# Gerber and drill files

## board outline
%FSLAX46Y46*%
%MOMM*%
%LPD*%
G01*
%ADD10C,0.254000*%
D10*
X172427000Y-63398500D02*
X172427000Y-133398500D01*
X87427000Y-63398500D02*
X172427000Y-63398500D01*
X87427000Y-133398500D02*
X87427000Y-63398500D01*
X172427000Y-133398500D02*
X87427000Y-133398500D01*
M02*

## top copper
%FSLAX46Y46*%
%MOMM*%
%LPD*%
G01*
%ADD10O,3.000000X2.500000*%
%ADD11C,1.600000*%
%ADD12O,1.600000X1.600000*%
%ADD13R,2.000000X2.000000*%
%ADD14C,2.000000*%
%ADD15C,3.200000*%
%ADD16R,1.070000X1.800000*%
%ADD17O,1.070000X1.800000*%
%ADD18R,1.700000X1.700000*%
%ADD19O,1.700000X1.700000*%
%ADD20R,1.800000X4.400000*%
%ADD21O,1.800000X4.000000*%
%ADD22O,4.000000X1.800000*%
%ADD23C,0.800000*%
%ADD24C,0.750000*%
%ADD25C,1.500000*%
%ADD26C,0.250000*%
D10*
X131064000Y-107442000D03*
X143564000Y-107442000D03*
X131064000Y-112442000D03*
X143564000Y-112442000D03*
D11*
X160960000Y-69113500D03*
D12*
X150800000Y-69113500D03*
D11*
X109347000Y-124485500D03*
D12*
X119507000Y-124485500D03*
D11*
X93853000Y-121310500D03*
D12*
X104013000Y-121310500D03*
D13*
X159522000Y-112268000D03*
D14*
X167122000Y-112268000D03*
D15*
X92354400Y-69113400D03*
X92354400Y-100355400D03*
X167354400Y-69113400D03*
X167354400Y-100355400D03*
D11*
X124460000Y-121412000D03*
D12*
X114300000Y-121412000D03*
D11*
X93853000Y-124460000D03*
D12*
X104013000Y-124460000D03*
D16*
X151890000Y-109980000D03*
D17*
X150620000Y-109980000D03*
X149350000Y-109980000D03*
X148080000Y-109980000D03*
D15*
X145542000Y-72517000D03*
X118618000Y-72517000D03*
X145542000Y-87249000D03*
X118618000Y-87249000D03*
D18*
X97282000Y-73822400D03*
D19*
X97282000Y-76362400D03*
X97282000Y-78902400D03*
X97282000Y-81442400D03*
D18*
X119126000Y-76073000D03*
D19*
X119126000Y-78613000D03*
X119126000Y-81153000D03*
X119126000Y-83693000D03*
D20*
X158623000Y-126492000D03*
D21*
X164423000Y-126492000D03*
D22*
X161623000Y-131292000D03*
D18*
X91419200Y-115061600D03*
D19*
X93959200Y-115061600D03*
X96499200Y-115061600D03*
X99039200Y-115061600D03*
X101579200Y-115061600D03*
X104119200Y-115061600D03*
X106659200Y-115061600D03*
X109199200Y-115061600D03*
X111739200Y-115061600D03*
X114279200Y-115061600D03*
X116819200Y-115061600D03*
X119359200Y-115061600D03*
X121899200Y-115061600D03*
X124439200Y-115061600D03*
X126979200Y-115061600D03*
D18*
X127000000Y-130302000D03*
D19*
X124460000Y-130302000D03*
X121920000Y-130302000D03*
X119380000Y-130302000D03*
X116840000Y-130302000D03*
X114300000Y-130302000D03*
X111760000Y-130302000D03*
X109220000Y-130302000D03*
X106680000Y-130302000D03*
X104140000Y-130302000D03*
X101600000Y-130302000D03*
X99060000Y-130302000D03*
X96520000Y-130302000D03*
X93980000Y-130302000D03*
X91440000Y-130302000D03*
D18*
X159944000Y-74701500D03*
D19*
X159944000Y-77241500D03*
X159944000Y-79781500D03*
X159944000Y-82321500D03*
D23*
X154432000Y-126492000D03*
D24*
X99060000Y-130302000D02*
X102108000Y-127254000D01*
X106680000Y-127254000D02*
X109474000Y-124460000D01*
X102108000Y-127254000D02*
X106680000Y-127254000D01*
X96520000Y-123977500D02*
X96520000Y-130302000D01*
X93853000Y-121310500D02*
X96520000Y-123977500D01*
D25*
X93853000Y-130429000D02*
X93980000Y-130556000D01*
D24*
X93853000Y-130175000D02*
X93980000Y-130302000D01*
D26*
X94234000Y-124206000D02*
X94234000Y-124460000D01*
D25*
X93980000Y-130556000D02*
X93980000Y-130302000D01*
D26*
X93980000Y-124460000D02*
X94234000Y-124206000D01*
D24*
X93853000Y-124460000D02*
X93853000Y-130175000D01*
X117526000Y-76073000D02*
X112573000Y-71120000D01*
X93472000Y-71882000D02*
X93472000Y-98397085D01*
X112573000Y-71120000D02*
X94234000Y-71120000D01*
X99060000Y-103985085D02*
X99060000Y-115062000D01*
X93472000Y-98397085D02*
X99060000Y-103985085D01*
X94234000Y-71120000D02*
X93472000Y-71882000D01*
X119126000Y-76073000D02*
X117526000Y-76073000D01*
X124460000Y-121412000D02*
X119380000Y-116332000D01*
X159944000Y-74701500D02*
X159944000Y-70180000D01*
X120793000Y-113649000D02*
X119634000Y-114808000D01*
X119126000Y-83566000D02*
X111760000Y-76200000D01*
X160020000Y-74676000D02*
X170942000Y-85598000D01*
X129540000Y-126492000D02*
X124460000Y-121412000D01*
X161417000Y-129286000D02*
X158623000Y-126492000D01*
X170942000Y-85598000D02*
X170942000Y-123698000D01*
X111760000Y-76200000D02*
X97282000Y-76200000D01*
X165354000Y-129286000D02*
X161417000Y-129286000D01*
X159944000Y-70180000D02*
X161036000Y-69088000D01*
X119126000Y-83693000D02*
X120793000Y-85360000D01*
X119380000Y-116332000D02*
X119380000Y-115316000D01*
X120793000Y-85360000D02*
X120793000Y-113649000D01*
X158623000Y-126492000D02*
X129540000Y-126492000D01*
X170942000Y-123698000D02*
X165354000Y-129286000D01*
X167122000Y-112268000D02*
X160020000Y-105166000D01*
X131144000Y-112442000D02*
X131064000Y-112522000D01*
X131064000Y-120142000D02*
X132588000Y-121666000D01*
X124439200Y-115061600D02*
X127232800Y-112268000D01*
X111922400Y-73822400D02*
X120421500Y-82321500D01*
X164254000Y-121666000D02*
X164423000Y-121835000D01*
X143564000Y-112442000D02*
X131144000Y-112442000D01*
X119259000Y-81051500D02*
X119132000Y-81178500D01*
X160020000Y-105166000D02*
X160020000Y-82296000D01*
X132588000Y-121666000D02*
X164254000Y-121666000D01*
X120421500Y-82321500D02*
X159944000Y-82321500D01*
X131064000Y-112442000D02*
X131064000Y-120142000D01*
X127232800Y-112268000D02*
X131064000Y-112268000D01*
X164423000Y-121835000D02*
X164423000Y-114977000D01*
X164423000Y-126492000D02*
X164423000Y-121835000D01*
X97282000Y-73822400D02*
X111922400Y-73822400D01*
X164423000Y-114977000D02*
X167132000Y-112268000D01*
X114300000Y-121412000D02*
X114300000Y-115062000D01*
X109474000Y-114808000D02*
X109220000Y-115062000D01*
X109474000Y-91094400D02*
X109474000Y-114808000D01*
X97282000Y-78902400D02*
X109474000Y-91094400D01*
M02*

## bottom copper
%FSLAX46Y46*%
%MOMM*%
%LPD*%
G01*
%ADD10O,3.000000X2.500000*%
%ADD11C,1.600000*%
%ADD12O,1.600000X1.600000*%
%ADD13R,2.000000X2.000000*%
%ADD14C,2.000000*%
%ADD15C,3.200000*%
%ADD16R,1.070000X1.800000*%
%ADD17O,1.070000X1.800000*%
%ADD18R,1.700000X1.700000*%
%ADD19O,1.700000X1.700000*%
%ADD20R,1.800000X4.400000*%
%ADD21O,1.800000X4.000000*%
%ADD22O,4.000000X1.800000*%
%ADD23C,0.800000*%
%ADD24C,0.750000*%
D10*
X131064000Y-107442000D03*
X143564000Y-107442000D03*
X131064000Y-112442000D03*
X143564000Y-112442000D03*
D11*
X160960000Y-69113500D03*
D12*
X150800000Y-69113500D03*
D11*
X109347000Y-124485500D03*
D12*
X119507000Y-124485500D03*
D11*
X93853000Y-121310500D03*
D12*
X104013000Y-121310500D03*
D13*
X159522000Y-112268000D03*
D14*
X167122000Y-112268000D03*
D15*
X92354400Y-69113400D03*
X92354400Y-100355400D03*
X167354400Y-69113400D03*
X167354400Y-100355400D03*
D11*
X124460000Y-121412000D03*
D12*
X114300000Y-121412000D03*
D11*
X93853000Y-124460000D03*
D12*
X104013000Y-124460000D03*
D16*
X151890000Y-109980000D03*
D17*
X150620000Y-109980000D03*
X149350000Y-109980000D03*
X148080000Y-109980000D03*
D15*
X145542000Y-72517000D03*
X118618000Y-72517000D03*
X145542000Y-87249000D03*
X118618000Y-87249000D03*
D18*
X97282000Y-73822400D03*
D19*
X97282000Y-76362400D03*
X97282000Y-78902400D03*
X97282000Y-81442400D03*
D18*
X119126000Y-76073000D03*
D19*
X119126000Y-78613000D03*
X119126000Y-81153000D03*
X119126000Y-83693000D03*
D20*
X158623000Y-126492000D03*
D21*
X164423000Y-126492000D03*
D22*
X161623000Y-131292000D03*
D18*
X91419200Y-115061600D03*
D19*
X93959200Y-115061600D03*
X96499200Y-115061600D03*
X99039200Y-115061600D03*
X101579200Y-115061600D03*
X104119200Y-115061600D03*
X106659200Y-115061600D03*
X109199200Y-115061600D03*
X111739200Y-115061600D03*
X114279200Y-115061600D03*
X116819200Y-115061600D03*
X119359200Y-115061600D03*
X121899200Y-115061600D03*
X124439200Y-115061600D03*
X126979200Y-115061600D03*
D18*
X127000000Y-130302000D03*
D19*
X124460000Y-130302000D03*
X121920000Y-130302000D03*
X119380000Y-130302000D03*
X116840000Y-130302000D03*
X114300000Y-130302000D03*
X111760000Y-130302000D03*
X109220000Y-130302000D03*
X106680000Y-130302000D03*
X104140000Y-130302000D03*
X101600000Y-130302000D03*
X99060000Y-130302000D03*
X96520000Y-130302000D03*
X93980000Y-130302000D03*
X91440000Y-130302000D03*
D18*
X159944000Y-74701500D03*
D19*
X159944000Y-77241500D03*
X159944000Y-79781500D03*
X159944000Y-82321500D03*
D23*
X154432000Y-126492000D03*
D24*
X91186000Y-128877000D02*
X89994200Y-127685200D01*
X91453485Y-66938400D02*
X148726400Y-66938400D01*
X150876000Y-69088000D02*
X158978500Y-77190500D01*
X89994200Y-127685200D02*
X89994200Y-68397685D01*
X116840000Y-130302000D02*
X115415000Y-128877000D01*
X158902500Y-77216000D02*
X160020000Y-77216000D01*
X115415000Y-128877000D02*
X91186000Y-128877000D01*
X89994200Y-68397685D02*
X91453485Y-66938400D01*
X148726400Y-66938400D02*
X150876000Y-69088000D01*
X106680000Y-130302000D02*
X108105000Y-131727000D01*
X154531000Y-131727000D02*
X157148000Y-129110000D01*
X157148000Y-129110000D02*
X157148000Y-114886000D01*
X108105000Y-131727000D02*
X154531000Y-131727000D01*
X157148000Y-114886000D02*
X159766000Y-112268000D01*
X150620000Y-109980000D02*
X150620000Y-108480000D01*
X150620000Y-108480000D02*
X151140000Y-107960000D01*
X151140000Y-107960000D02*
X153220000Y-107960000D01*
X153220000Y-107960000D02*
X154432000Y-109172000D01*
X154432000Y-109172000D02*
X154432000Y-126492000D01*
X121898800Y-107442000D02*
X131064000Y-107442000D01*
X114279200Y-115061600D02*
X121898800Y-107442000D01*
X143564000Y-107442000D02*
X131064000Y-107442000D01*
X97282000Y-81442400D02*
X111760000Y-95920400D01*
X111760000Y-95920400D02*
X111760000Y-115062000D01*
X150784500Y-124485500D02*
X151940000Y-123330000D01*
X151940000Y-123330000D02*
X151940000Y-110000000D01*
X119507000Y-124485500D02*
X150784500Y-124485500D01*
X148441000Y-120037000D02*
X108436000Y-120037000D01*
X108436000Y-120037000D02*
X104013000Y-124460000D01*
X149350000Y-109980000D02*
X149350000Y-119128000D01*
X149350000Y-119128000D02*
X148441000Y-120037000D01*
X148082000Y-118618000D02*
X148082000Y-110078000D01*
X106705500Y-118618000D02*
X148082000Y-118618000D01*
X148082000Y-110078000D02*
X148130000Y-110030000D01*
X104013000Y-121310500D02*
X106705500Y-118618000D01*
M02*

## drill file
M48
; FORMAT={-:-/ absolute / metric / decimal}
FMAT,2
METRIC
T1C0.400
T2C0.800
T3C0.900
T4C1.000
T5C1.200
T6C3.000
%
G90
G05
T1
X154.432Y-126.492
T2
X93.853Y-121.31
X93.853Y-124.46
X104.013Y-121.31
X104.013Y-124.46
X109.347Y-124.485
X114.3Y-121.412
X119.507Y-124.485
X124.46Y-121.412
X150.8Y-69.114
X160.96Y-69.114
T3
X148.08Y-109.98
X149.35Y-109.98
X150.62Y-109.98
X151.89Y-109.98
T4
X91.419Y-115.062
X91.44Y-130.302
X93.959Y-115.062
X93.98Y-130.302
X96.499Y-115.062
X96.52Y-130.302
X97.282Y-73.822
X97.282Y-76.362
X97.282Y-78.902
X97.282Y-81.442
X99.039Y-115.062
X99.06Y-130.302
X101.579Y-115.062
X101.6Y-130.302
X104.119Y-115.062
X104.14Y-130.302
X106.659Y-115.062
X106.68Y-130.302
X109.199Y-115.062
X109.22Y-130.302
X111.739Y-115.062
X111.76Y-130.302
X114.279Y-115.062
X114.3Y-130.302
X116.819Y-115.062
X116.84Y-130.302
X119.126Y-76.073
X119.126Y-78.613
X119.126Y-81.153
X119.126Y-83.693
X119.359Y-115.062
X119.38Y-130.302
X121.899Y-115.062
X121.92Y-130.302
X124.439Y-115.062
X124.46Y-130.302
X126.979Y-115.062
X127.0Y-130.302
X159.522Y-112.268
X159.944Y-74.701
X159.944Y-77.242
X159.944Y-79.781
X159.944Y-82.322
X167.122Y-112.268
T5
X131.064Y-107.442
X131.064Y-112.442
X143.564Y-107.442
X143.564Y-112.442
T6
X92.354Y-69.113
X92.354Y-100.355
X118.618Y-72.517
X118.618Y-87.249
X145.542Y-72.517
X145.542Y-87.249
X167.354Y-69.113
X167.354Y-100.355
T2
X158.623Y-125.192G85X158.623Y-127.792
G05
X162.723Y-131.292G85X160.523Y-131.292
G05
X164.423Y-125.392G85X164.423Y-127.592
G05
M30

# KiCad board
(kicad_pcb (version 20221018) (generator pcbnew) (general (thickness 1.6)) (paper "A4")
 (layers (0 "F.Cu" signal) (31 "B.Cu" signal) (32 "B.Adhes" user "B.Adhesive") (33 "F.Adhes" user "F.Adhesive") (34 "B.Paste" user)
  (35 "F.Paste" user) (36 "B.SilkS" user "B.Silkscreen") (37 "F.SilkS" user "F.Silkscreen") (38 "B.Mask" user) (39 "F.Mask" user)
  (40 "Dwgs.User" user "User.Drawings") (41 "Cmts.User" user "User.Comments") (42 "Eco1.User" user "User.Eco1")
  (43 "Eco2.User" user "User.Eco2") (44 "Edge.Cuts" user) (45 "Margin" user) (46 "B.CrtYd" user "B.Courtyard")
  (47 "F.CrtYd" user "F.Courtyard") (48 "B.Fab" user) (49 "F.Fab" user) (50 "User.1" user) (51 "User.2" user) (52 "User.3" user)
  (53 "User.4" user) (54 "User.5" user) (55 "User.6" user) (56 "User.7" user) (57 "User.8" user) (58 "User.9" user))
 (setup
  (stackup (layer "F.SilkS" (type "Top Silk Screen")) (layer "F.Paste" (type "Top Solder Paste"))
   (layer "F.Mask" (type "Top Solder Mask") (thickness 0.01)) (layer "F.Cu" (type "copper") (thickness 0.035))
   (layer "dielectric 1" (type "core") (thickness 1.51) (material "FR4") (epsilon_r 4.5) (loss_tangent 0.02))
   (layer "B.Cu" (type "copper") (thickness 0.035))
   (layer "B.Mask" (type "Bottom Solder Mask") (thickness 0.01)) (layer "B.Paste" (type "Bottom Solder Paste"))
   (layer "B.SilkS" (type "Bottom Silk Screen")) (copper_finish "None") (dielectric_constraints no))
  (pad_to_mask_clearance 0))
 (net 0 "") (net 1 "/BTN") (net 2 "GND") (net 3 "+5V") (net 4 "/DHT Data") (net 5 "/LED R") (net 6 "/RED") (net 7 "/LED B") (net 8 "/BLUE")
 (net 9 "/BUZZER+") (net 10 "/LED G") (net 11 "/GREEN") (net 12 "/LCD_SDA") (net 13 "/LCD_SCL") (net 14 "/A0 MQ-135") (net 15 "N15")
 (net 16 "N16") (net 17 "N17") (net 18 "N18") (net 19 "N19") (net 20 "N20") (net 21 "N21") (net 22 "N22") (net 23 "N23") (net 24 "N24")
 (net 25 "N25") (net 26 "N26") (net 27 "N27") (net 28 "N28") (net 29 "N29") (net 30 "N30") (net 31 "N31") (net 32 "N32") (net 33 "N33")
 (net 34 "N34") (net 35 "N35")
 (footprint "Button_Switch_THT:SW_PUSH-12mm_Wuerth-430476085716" (layer "F.Cu") (at 131.064 107.442)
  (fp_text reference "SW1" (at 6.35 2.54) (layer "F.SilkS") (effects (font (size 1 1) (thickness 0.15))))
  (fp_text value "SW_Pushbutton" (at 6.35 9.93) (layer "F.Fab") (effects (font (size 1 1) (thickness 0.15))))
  (pad "1" thru_hole oval (at 0 0) (size 3 2.5) (drill 1.2) (layers "*.Cu" "*.Mask") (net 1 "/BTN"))
  (pad "1" thru_hole oval (at 12.5 0) (size 3 2.5) (drill 1.2) (layers "*.Cu" "*.Mask") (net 1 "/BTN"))
  (pad "2" thru_hole oval (at 0 5) (size 3 2.5) (drill 1.2) (layers "*.Cu" "*.Mask") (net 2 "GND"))
  (pad "2" thru_hole oval (at 12.5 5) (size 3 2.5) (drill 1.2) (layers "*.Cu" "*.Mask") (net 2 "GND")))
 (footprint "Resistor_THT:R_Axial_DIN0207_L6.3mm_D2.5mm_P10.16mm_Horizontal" (layer "F.Cu") (at 160.96 69.1135 180)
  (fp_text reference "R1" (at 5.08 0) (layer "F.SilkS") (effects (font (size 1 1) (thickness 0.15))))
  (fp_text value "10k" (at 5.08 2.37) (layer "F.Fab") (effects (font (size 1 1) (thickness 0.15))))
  (pad "1" thru_hole circle (at 0 0 180) (size 1.6 1.6) (drill 0.8) (layers "*.Cu" "*.Mask") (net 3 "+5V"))
  (pad "2" thru_hole oval (at 10.16 0 180) (size 1.6 1.6) (drill 0.8) (layers "*.Cu" "*.Mask") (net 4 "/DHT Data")))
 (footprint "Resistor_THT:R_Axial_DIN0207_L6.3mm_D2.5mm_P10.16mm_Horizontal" (layer "F.Cu") (at 109.347 124.4855)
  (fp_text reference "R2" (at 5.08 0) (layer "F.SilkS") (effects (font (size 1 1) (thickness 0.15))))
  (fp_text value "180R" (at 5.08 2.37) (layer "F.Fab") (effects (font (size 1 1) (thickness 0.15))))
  (pad "1" thru_hole circle (at 0 0) (size 1.6 1.6) (drill 0.8) (layers "*.Cu" "*.Mask") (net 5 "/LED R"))
  (pad "2" thru_hole oval (at 10.16 0) (size 1.6 1.6) (drill 0.8) (layers "*.Cu" "*.Mask") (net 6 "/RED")))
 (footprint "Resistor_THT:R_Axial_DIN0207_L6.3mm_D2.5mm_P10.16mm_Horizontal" (layer "F.Cu") (at 93.853 121.3105)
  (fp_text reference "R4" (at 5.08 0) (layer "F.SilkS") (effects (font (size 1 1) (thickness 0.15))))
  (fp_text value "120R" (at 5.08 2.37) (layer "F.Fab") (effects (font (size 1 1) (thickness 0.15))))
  (pad "1" thru_hole circle (at 0 0) (size 1.6 1.6) (drill 0.8) (layers "*.Cu" "*.Mask") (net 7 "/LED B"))
  (pad "2" thru_hole oval (at 10.16 0) (size 1.6 1.6) (drill 0.8) (layers "*.Cu" "*.Mask") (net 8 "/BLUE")))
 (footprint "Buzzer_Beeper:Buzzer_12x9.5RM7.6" (layer "F.Cu") (at 159.522 112.268)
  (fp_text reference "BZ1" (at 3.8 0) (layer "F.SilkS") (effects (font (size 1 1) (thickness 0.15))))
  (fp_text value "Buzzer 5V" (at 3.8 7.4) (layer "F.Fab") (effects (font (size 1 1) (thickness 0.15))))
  (pad "1" thru_hole rect (at 0 0) (size 2 2) (drill 1) (layers "*.Cu" "*.Mask") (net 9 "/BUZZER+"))
  (pad "2" thru_hole circle (at 7.6 0) (size 2 2) (drill 1) (layers "*.Cu" "*.Mask") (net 2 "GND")))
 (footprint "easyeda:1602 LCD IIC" (layer "F.Cu") (at 89.8144 66.8274)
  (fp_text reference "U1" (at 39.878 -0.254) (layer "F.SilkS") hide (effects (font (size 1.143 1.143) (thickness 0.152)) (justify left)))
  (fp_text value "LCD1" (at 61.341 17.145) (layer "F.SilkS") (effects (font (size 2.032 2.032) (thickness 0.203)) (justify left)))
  (pad "" thru_hole circle (at 2.54 2.286) (size 3.2 3.2) (drill 3) (layers "*.Cu" "*.Mask"))
  (pad "" thru_hole circle (at 2.54 33.528) (size 3.2 3.2) (drill 3) (layers "*.Cu" "*.Mask"))
  (pad "" thru_hole circle (at 77.54 2.286) (size 3.2 3.2) (drill 3) (layers "*.Cu" "*.Mask"))
  (pad "" thru_hole circle (at 77.54 33.528) (size 3.2 3.2) (drill 3) (layers "*.Cu" "*.Mask")))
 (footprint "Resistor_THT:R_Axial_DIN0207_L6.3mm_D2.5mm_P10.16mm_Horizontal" (layer "F.Cu") (at 124.46 121.412 180)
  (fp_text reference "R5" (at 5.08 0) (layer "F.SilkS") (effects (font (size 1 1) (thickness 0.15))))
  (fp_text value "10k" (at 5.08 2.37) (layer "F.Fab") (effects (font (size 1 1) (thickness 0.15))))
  (pad "1" thru_hole circle (at 0 0 180) (size 1.6 1.6) (drill 0.8) (layers "*.Cu" "*.Mask") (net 3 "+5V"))
  (pad "2" thru_hole oval (at 10.16 0 180) (size 1.6 1.6) (drill 0.8) (layers "*.Cu" "*.Mask") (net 1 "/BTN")))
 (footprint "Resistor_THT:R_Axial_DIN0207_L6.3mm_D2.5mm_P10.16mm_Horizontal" (layer "F.Cu") (at 93.853 124.46)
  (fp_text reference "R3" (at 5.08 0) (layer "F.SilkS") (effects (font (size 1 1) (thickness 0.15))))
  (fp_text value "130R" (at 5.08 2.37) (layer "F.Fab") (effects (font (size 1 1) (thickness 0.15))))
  (pad "1" thru_hole circle (at 0 0) (size 1.6 1.6) (drill 0.8) (layers "*.Cu" "*.Mask") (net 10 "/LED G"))
  (pad "2" thru_hole oval (at 10.16 0) (size 1.6 1.6) (drill 0.8) (layers "*.Cu" "*.Mask") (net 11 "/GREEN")))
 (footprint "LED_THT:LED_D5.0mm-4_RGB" (layer "F.Cu") (at 151.89 109.98 180)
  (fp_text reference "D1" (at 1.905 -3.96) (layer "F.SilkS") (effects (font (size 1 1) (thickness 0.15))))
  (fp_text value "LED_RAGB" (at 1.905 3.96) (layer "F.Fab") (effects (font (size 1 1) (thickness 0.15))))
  (pad "1" thru_hole rect (at 0 0 180) (size 1.07 1.8) (drill 0.9) (layers "*.Cu" "*.Mask") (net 6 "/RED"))
  (pad "2" thru_hole oval (at 1.27 0 180) (size 1.07 1.8) (drill 0.9) (layers "*.Cu" "*.Mask") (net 3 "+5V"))
  (pad "3" thru_hole oval (at 2.54 0 180) (size 1.07 1.8) (drill 0.9) (layers "*.Cu" "*.Mask") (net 11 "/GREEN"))
  (pad "4" thru_hole oval (at 3.81 0 180) (size 1.07 1.8) (drill 0.9) (layers "*.Cu" "*.Mask") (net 8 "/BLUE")))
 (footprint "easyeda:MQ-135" (layer "F.Cu") (at 118.618 87.249 -90)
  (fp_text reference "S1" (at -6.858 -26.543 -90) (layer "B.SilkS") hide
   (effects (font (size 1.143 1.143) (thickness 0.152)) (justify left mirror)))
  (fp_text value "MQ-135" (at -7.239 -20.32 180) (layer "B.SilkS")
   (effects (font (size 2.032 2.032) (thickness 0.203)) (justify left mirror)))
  (pad "" thru_hole circle (at -14.732 -26.924) (size 3.2 3.2) (drill 3) (layers "*.Cu" "*.Mask"))
  (pad "" thru_hole circle (at -14.732 0) (size 3.2 3.2) (drill 3) (layers "*.Cu" "*.Mask"))
  (pad "" thru_hole circle (at 0 -26.924) (size 3.2 3.2) (drill 3) (layers "*.Cu" "*.Mask"))
  (pad "" thru_hole circle (at 0 0) (size 3.2 3.2) (drill 3) (layers "*.Cu" "*.Mask")))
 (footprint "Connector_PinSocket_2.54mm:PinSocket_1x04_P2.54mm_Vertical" (layer "F.Cu") (at 97.282 73.8224)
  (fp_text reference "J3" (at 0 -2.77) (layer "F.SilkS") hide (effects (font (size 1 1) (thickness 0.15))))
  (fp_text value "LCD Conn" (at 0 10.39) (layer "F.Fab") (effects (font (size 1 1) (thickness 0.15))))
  (pad "1" thru_hole rect (at 0 0) (size 1.7 1.7) (drill 1) (layers "*.Cu" "*.Mask") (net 2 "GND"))
  (pad "2" thru_hole oval (at 0 2.54) (size 1.7 1.7) (drill 1) (layers "*.Cu" "*.Mask") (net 3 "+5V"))
  (pad "3" thru_hole oval (at 0 5.08) (size 1.7 1.7) (drill 1) (layers "*.Cu" "*.Mask") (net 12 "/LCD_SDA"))
  (pad "4" thru_hole oval (at 0 7.62) (size 1.7 1.7) (drill 1) (layers "*.Cu" "*.Mask") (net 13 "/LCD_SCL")))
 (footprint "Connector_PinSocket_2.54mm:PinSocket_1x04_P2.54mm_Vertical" (layer "B.Cu") (at 119.126 76.073 180)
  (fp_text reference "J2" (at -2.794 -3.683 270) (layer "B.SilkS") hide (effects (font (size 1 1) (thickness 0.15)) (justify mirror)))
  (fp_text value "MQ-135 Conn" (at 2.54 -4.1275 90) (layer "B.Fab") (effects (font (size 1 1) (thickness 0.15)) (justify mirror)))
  (pad "1" thru_hole rect (at 0 0 180) (size 1.7 1.7) (drill 1) (layers "*.Cu" "*.Mask") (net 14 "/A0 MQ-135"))
  (pad "2" thru_hole oval (at 0 -2.54 180) (size 1.7 1.7) (drill 1) (layers "*.Cu" "*.Mask") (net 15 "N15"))
  (pad "3" thru_hole oval (at 0 -5.08 180) (size 1.7 1.7) (drill 1) (layers "*.Cu" "*.Mask") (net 2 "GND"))
  (pad "4" thru_hole oval (at 0 -7.62 180) (size 1.7 1.7) (drill 1) (layers "*.Cu" "*.Mask") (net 3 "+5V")))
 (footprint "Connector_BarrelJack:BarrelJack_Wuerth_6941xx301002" (layer "B.Cu") (at 158.623 126.492 -90)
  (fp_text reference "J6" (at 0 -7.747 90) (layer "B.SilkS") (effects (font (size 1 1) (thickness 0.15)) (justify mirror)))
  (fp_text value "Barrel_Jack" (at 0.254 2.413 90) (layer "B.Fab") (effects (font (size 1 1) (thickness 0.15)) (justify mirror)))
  (pad "1" thru_hole rect (at 0 0 270) (size 4.4 1.8) (drill oval 3.4 0.8) (layers "*.Cu" "*.Mask") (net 3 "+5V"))
  (pad "2" thru_hole oval (at 0 -5.8 270) (size 4 1.8) (drill oval 3 0.8) (layers "*.Cu" "*.Mask") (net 2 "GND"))
  (pad "3" thru_hole oval (at 4.8 -3 180) (size 4 1.8) (drill oval 3 0.8) (layers "*.Cu" "*.Mask")))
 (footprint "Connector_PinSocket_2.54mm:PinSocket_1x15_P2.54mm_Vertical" (layer "B.Cu") (at 91.4192 115.0616 -90)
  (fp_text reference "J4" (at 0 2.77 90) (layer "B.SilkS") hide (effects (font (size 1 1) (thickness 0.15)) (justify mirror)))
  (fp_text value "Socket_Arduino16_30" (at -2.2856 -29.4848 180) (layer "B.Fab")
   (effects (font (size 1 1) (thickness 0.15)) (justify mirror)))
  (pad "1" thru_hole rect (at 0 0 270) (size 1.7 1.7) (drill 1) (layers "*.Cu" "*.Mask") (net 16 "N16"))
  (pad "2" thru_hole oval (at 0 -2.54 270) (size 1.7 1.7) (drill 1) (layers "*.Cu" "*.Mask") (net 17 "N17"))
  (pad "3" thru_hole oval (at 0 -5.08 270) (size 1.7 1.7) (drill 1) (layers "*.Cu" "*.Mask") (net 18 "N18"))
  (pad "4" thru_hole oval (at 0 -7.62 270) (size 1.7 1.7) (drill 1) (layers "*.Cu" "*.Mask") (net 14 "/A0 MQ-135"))
  (pad "5" thru_hole oval (at 0 -10.16 270) (size 1.7 1.7) (drill 1) (layers "*.Cu" "*.Mask") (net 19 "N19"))
  (pad "6" thru_hole oval (at 0 -12.7 270) (size 1.7 1.7) (drill 1) (layers "*.Cu" "*.Mask") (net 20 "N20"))
  (pad "7" thru_hole oval (at 0 -15.24 270) (size 1.7 1.7) (drill 1) (layers "*.Cu" "*.Mask") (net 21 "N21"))
  (pad "8" thru_hole oval (at 0 -17.78 270) (size 1.7 1.7) (drill 1) (layers "*.Cu" "*.Mask") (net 12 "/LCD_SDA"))
  (pad "9" thru_hole oval (at 0 -20.32 270) (size 1.7 1.7) (drill 1) (layers "*.Cu" "*.Mask") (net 13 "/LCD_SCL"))
  (pad "10" thru_hole oval (at 0 -22.86 270) (size 1.7 1.7) (drill 1) (layers "*.Cu" "*.Mask") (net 1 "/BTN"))
  (pad "11" thru_hole oval (at 0 -25.4 270) (size 1.7 1.7) (drill 1) (layers "*.Cu" "*.Mask") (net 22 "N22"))
  (pad "12" thru_hole oval (at 0 -27.94 270) (size 1.7 1.7) (drill 1) (layers "*.Cu" "*.Mask") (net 3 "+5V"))
  (pad "13" thru_hole oval (at 0 -30.48 270) (size 1.7 1.7) (drill 1) (layers "*.Cu" "*.Mask") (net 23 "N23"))
  (pad "14" thru_hole oval (at 0 -33.02 270) (size 1.7 1.7) (drill 1) (layers "*.Cu" "*.Mask") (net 2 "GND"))
  (pad "15" thru_hole oval (at 0 -35.56 270) (size 1.7 1.7) (drill 1) (layers "*.Cu" "*.Mask") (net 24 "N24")))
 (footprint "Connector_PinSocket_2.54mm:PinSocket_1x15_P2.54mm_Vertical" (layer "B.Cu") (at 127 130.302 90)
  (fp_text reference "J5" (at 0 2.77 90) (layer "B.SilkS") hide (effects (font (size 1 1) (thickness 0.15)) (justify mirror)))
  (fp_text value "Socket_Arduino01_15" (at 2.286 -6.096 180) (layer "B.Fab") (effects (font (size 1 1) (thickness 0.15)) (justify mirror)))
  (pad "1" thru_hole rect (at 0 0 90) (size 1.7 1.7) (drill 1) (layers "*.Cu" "*.Mask") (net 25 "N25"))
  (pad "2" thru_hole oval (at 0 -2.54 90) (size 1.7 1.7) (drill 1) (layers "*.Cu" "*.Mask") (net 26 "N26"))
  (pad "3" thru_hole oval (at 0 -5.08 90) (size 1.7 1.7) (drill 1) (layers "*.Cu" "*.Mask") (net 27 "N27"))
  (pad "4" thru_hole oval (at 0 -7.62 90) (size 1.7 1.7) (drill 1) (layers "*.Cu" "*.Mask") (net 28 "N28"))
  (pad "5" thru_hole oval (at 0 -10.16 90) (size 1.7 1.7) (drill 1) (layers "*.Cu" "*.Mask") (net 4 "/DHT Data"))
  (pad "6" thru_hole oval (at 0 -12.7 90) (size 1.7 1.7) (drill 1) (layers "*.Cu" "*.Mask") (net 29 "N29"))
  (pad "7" thru_hole oval (at 0 -15.24 90) (size 1.7 1.7) (drill 1) (layers "*.Cu" "*.Mask") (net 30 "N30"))
  (pad "8" thru_hole oval (at 0 -17.78 90) (size 1.7 1.7) (drill 1) (layers "*.Cu" "*.Mask") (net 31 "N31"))
  (pad "9" thru_hole oval (at 0 -20.32 90) (size 1.7 1.7) (drill 1) (layers "*.Cu" "*.Mask") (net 9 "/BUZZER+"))
  (pad "10" thru_hole oval (at 0 -22.86 90) (size 1.7 1.7) (drill 1) (layers "*.Cu" "*.Mask") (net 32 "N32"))
  (pad "11" thru_hole oval (at 0 -25.4 90) (size 1.7 1.7) (drill 1) (layers "*.Cu" "*.Mask") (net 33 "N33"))
  (pad "12" thru_hole oval (at 0 -27.94 90) (size 1.7 1.7) (drill 1) (layers "*.Cu" "*.Mask") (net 5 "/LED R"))
  (pad "13" thru_hole oval (at 0 -30.48 90) (size 1.7 1.7) (drill 1) (layers "*.Cu" "*.Mask") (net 7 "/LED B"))
  (pad "14" thru_hole oval (at 0 -33.02 90) (size 1.7 1.7) (drill 1) (layers "*.Cu" "*.Mask") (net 10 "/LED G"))
  (pad "15" thru_hole oval (at 0 -35.56 90) (size 1.7 1.7) (drill 1) (layers "*.Cu" "*.Mask") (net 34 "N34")))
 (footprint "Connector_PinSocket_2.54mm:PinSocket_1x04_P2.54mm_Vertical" (layer "B.Cu") (at 159.944 74.7015 180)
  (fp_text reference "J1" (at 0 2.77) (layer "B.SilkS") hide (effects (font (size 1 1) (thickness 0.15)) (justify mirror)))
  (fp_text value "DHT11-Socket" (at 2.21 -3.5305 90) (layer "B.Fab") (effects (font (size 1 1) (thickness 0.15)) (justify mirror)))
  (pad "1" thru_hole rect (at 0 0 180) (size 1.7 1.7) (drill 1) (layers "*.Cu" "*.Mask") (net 3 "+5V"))
  (pad "2" thru_hole oval (at 0 -2.54 180) (size 1.7 1.7) (drill 1) (layers "*.Cu" "*.Mask") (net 4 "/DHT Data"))
  (pad "3" thru_hole oval (at 0 -5.08 180) (size 1.7 1.7) (drill 1) (layers "*.Cu" "*.Mask") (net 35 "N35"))
  (pad "4" thru_hole oval (at 0 -7.62 180) (size 1.7 1.7) (drill 1) (layers "*.Cu" "*.Mask") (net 2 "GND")))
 (gr_line (start 172.427 63.3985) (end 172.427 133.3985) (stroke (width 0.254) (type solid)) (layer "Edge.Cuts"))
 (gr_line (start 87.427 63.3985) (end 172.427 63.3985) (stroke (width 0.254) (type solid)) (layer "Edge.Cuts"))
 (gr_line (start 87.427 133.3985) (end 87.427 63.3985) (stroke (width 0.254) (type solid)) (layer "Edge.Cuts"))
 (gr_line (start 172.427 133.3985) (end 87.427 133.3985) (stroke (width 0.254) (type solid)) (layer "Edge.Cuts"))
 (segment (start 91.186 128.877) (end 89.9942 127.6852) (width 0.75) (layer "B.Cu") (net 4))
 (segment (start 91.453485 66.9384) (end 148.7264 66.9384) (width 0.75) (layer "B.Cu") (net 4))
 (segment (start 150.876 69.088) (end 158.9785 77.1905) (width 0.75) (layer "B.Cu") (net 4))
 (segment (start 89.9942 127.6852) (end 89.9942 68.397685) (width 0.75) (layer "B.Cu") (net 4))
 (segment (start 116.84 130.302) (end 115.415 128.877) (width 0.75) (layer "B.Cu") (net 4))
 (segment (start 158.9025 77.216) (end 160.02 77.216) (width 0.75) (layer "B.Cu") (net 4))
 (segment (start 115.415 128.877) (end 91.186 128.877) (width 0.75) (layer "B.Cu") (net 4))
 (segment (start 89.9942 68.397685) (end 91.453485 66.9384) (width 0.75) (layer "B.Cu") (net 4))
 (segment (start 148.7264 66.9384) (end 150.876 69.088) (width 0.75) (layer "B.Cu") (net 4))
 (segment (start 106.68 130.302) (end 108.105 131.727) (width 0.75) (layer "B.Cu") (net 9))
 (segment (start 154.531 131.727) (end 157.148 129.11) (width 0.75) (layer "B.Cu") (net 9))
 (segment (start 157.148 129.11) (end 157.148 114.886) (width 0.75) (layer "B.Cu") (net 9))
 (segment (start 108.105 131.727) (end 154.531 131.727) (width 0.75) (layer "B.Cu") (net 9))
 (segment (start 157.148 114.886) (end 159.766 112.268) (width 0.75) (layer "B.Cu") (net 9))
 (segment (start 99.06 130.302) (end 102.108 127.254) (width 0.75) (layer "F.Cu") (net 5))
 (segment (start 106.68 127.254) (end 109.474 124.46) (width 0.75) (layer "F.Cu") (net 5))
 (segment (start 102.108 127.254) (end 106.68 127.254) (width 0.75) (layer "F.Cu") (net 5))
 (segment (start 96.52 123.9775) (end 96.52 130.302) (width 0.75) (layer "F.Cu") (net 7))
 (segment (start 93.853 121.3105) (end 96.52 123.9775) (width 0.75) (layer "F.Cu") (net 7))
 (segment (start 93.853 130.429) (end 93.98 130.556) (width 1.5) (layer "F.Cu") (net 10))
 (segment (start 93.853 130.175) (end 93.98 130.302) (width 0.75) (layer "F.Cu") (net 10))
 (segment (start 94.234 124.206) (end 94.234 124.46) (width 0.25) (layer "F.Cu") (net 10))
 (segment (start 93.98 130.556) (end 93.98 130.302) (width 1.5) (layer "F.Cu") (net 10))
 (segment (start 93.98 124.46) (end 94.234 124.206) (width 0.25) (layer "F.Cu") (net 10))
 (segment (start 93.853 124.46) (end 93.853 130.175) (width 0.75) (layer "F.Cu") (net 10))
 (segment (start 117.526 76.073) (end 112.573 71.12) (width 0.75) (layer "F.Cu") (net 14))
 (segment (start 93.472 71.882) (end 93.472 98.397085) (width 0.75) (layer "F.Cu") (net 14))
 (segment (start 112.573 71.12) (end 94.234 71.12) (width 0.75) (layer "F.Cu") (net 14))
 (segment (start 99.06 103.985085) (end 99.06 115.062) (width 0.75) (layer "F.Cu") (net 14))
 (segment (start 93.472 98.397085) (end 99.06 103.985085) (width 0.75) (layer "F.Cu") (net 14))
 (segment (start 94.234 71.12) (end 93.472 71.882) (width 0.75) (layer "F.Cu") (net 14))
 (segment (start 119.126 76.073) (end 117.526 76.073) (width 0.75) (layer "F.Cu") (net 14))
 (segment (start 124.46 121.412) (end 119.38 116.332) (width 0.75) (layer "F.Cu") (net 3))
 (segment (start 159.944 74.7015) (end 159.944 70.18) (width 0.75) (layer "F.Cu") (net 3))
 (segment (start 120.793 113.649) (end 119.634 114.808) (width 0.75) (layer "F.Cu") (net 3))
 (segment (start 119.126 83.566) (end 111.76 76.2) (width 0.75) (layer "F.Cu") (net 3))
 (segment (start 160.02 74.676) (end 170.942 85.598) (width 0.75) (layer "F.Cu") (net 3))
 (segment (start 129.54 126.492) (end 124.46 121.412) (width 0.75) (layer "F.Cu") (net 3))
 (segment (start 161.417 129.286) (end 158.623 126.492) (width 0.75) (layer "F.Cu") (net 3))
 (segment (start 170.942 85.598) (end 170.942 123.698) (width 0.75) (layer "F.Cu") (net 3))
 (segment (start 111.76 76.2) (end 97.282 76.2) (width 0.75) (layer "F.Cu") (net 3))
 (segment (start 165.354 129.286) (end 161.417 129.286) (width 0.75) (layer "F.Cu") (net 3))
 (segment (start 159.944 70.18) (end 161.036 69.088) (width 0.75) (layer "F.Cu") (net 3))
 (segment (start 119.126 83.693) (end 120.793 85.36) (width 0.75) (layer "F.Cu") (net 3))
 (segment (start 119.38 116.332) (end 119.38 115.316) (width 0.75) (layer "F.Cu") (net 3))
 (segment (start 120.793 85.36) (end 120.793 113.649) (width 0.75) (layer "F.Cu") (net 3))
 (segment (start 158.623 126.492) (end 129.54 126.492) (width 0.75) (layer "F.Cu") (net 3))
 (segment (start 170.942 123.698) (end 165.354 129.286) (width 0.75) (layer "F.Cu") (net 3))
 (via (at 154.432 126.492) (size 0.8) (drill 0.4) (layers "F.Cu" "B.Cu") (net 3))
 (segment (start 150.62 109.98) (end 150.62 108.48) (width 0.75) (layer "B.Cu") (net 3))
 (segment (start 150.62 108.48) (end 151.14 107.96) (width 0.75) (layer "B.Cu") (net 3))
 (segment (start 151.14 107.96) (end 153.22 107.96) (width 0.75) (layer "B.Cu") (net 3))
 (segment (start 153.22 107.96) (end 154.432 109.172) (width 0.75) (layer "B.Cu") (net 3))
 (segment (start 154.432 109.172) (end 154.432 126.492) (width 0.75) (layer "B.Cu") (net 3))
 (segment (start 167.122 112.268) (end 160.02 105.166) (width 0.75) (layer "F.Cu") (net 2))
 (segment (start 131.144 112.442) (end 131.064 112.522) (width 0.75) (layer "F.Cu") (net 2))
 (segment (start 131.064 120.142) (end 132.588 121.666) (width 0.75) (layer "F.Cu") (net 2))
 (segment (start 124.4392 115.0616) (end 127.2328 112.268) (width 0.75) (layer "F.Cu") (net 2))
 (segment (start 111.9224 73.8224) (end 120.4215 82.3215) (width 0.75) (layer "F.Cu") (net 2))
 (segment (start 164.254 121.666) (end 164.423 121.835) (width 0.75) (layer "F.Cu") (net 2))
 (segment (start 143.564 112.442) (end 131.144 112.442) (width 0.75) (layer "F.Cu") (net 2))
 (segment (start 119.259 81.0515) (end 119.132 81.1785) (width 0.75) (layer "F.Cu") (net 2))
 (segment (start 160.02 105.166) (end 160.02 82.296) (width 0.75) (layer "F.Cu") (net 2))
 (segment (start 132.588 121.666) (end 164.254 121.666) (width 0.75) (layer "F.Cu") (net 2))
 (segment (start 120.4215 82.3215) (end 159.944 82.3215) (width 0.75) (layer "F.Cu") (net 2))
 (segment (start 131.064 112.442) (end 131.064 120.142) (width 0.75) (layer "F.Cu") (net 2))
 (segment (start 127.2328 112.268) (end 131.064 112.268) (width 0.75) (layer "F.Cu") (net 2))
 (segment (start 164.423 121.835) (end 164.423 114.977) (width 0.75) (layer "F.Cu") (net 2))
 (segment (start 164.423 126.492) (end 164.423 121.835) (width 0.75) (layer "F.Cu") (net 2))
 (segment (start 97.282 73.8224) (end 111.9224 73.8224) (width 0.75) (layer "F.Cu") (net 2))
 (segment (start 164.423 114.977) (end 167.132 112.268) (width 0.75) (layer "F.Cu") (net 2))
 (segment (start 114.3 121.412) (end 114.3 115.062) (width 0.75) (layer "F.Cu") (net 1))
 (segment (start 121.8988 107.442) (end 131.064 107.442) (width 0.75) (layer "B.Cu") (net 1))
 (segment (start 114.2792 115.0616) (end 121.8988 107.442) (width 0.75) (layer "B.Cu") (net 1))
 (segment (start 143.564 107.442) (end 131.064 107.442) (width 0.75) (layer "B.Cu") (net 1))
 (segment (start 109.474 114.808) (end 109.22 115.062) (width 0.75) (layer "F.Cu") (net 12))
 (segment (start 109.474 91.0944) (end 109.474 114.808) (width 0.75) (layer "F.Cu") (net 12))
 (segment (start 97.282 78.9024) (end 109.474 91.0944) (width 0.75) (layer "F.Cu") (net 12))
 (segment (start 97.282 81.4424) (end 111.76 95.9204) (width 0.75) (layer "B.Cu") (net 13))
 (segment (start 111.76 95.9204) (end 111.76 115.062) (width 0.75) (layer "B.Cu") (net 13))
 (segment (start 150.7845 124.4855) (end 151.94 123.33) (width 0.75) (layer "B.Cu") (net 6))
 (segment (start 151.94 123.33) (end 151.94 110) (width 0.75) (layer "B.Cu") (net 6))
 (segment (start 119.507 124.4855) (end 150.7845 124.4855) (width 0.75) (layer "B.Cu") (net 6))
 (segment (start 148.441 120.037) (end 108.436 120.037) (width 0.75) (layer "B.Cu") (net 11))
 (segment (start 108.436 120.037) (end 104.013 124.46) (width 0.75) (layer "B.Cu") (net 11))
 (segment (start 149.35 109.98) (end 149.35 119.128) (width 0.75) (layer "B.Cu") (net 11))
 (segment (start 149.35 119.128) (end 148.441 120.037) (width 0.75) (layer "B.Cu") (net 11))
 (segment (start 148.082 118.618) (end 148.082 110.078) (width 0.75) (layer "B.Cu") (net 8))
 (segment (start 106.7055 118.618) (end 148.082 118.618) (width 0.75) (layer "B.Cu") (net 8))
 (segment (start 148.082 110.078) (end 148.13 110.03) (width 0.75) (layer "B.Cu") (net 8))
 (segment (start 104.013 121.3105) (end 106.7055 118.618) (width 0.75) (layer "B.Cu") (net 8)))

